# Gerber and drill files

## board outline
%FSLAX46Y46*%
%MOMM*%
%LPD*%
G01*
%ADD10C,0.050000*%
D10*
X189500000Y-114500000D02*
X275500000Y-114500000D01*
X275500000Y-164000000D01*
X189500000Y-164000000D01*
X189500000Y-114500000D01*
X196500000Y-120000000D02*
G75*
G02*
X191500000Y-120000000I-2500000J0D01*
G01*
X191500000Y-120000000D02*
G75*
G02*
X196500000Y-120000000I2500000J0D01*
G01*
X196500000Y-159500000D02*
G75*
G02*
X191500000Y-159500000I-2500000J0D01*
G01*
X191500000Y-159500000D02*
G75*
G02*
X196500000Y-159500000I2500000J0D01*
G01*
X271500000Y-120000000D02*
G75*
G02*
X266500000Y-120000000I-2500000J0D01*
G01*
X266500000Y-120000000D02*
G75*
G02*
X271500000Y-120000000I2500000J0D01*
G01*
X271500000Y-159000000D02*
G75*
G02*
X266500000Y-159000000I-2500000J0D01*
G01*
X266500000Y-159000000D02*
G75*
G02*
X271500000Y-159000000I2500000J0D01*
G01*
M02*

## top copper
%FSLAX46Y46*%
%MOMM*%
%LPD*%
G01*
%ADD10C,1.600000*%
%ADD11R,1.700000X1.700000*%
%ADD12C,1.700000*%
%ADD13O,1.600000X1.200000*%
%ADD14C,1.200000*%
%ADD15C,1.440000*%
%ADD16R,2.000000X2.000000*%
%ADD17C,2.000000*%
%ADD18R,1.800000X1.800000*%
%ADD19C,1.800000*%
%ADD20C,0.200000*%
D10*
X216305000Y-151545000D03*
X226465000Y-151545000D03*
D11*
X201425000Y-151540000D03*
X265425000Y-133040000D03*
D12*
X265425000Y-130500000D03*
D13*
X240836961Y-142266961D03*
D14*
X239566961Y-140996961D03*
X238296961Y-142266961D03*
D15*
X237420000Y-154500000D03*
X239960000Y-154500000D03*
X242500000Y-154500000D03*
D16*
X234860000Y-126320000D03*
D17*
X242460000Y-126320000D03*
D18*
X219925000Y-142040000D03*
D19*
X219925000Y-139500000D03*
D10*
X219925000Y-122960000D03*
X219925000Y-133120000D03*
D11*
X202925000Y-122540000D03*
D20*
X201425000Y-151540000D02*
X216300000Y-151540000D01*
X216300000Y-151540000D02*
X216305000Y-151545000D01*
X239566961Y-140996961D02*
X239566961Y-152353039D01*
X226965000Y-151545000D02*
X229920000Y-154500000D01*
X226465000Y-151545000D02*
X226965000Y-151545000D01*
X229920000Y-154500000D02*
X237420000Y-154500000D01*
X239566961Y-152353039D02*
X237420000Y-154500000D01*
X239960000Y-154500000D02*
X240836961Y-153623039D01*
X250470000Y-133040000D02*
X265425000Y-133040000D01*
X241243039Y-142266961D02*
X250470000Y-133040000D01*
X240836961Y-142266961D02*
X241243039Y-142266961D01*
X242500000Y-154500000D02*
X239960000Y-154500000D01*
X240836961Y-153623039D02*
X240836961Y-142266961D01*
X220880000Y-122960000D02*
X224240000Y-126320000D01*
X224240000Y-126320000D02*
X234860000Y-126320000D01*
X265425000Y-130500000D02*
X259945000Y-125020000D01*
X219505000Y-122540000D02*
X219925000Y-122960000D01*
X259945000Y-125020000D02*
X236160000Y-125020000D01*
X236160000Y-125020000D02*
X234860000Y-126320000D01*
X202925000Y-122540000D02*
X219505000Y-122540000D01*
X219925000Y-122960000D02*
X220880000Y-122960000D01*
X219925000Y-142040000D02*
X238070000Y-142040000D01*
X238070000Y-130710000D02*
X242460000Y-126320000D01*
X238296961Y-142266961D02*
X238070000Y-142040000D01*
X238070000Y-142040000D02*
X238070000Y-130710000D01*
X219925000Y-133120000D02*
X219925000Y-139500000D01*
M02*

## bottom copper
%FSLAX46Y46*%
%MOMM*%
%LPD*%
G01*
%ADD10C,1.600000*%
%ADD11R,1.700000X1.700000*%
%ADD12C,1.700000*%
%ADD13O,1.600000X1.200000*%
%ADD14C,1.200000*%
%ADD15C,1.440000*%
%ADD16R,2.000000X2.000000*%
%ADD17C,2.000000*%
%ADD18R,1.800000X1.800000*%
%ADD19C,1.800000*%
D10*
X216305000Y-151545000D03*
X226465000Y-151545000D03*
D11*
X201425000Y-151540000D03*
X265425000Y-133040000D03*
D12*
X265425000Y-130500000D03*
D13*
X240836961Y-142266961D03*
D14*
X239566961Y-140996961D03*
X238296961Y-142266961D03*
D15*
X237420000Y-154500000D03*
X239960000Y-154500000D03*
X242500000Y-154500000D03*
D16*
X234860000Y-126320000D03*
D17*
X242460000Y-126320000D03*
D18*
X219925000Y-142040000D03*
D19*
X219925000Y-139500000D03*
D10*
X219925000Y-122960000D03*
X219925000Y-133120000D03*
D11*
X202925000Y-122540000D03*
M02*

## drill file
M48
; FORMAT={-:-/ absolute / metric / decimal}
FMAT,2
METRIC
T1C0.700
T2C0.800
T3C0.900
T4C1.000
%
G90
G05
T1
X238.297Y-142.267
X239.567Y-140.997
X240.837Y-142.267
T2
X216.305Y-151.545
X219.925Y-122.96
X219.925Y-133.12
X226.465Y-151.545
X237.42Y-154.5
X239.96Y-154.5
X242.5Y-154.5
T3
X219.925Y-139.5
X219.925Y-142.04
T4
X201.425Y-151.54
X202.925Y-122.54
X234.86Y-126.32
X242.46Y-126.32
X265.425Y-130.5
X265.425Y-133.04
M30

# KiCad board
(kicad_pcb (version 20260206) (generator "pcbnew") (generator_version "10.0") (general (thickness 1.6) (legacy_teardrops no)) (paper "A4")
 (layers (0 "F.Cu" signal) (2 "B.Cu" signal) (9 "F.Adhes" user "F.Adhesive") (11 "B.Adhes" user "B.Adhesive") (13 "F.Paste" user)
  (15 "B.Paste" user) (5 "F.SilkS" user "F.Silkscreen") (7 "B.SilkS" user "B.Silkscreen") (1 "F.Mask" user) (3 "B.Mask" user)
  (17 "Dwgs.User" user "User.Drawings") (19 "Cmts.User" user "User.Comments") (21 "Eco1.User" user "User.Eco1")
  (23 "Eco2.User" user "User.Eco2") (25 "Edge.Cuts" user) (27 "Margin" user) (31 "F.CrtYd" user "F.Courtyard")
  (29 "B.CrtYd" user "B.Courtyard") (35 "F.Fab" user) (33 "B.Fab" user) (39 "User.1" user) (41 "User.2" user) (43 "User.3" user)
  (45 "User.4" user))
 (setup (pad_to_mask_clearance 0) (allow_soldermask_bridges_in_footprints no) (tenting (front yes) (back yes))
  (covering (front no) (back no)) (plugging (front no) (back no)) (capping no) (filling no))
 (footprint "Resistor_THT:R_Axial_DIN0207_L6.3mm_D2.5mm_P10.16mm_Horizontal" (layer "F.Cu") (at 216.305 151.545)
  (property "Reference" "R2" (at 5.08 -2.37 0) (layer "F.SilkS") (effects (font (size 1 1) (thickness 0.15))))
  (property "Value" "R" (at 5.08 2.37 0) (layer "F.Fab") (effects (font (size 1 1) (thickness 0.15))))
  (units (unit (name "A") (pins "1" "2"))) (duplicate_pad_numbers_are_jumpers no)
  (pad "1" thru_hole circle (at 0 0) (size 1.6 1.6) (drill 0.8) (layers "*.Cu" "*.Mask") (remove_unused_layers no) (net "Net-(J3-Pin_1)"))
  (pad "2" thru_hole circle (at 10.16 0) (size 1.6 1.6) (drill 0.8) (layers "*.Cu" "*.Mask") (remove_unused_layers no) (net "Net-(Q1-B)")))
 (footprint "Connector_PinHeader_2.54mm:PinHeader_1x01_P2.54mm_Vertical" (layer "F.Cu") (at 201.425 151.54)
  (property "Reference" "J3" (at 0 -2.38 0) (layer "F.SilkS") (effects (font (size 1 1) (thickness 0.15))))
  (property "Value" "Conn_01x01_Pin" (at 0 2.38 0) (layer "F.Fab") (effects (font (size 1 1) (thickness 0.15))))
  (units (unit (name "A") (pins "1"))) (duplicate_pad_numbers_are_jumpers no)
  (pad "1" thru_hole rect (at 0 0) (size 1.7 1.7) (drill 1) (layers "*.Cu" "*.Mask") (remove_unused_layers no) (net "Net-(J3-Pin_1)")))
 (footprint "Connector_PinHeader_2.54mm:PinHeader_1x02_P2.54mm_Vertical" (layer "F.Cu") (at 265.425 133.04 180)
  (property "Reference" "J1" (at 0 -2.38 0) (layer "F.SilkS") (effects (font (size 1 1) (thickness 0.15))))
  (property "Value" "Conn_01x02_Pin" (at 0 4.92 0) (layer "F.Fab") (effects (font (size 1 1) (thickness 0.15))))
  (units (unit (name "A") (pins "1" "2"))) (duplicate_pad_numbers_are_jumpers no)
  (pad "1" thru_hole rect (at 0 0 180) (size 1.7 1.7) (drill 1) (layers "*.Cu" "*.Mask") (remove_unused_layers no) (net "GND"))
  (pad "2" thru_hole circle (at 0 2.54 180) (size 1.7 1.7) (drill 1) (layers "*.Cu" "*.Mask") (remove_unused_layers no) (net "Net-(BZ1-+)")))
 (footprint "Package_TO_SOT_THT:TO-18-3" (layer "F.Cu") (at 240.836961 142.266961 180)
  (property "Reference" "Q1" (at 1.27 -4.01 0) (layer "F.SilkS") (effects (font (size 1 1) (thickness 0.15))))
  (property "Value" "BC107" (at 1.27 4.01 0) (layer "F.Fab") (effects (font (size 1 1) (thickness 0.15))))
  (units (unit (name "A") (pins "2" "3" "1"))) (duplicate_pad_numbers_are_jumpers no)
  (pad "1" thru_hole oval (at 0 0 180) (size 1.6 1.2) (drill 0.7) (layers "*.Cu" "*.Mask") (remove_unused_layers no) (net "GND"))
  (pad "2" thru_hole circle (at 1.27 1.27 180) (size 1.2 1.2) (drill 0.7) (layers "*.Cu" "*.Mask") (remove_unused_layers no)
   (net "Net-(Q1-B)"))
  (pad "3" thru_hole circle (at 2.54 0 180) (size 1.2 1.2) (drill 0.7) (layers "*.Cu" "*.Mask") (remove_unused_layers no)
   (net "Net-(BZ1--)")))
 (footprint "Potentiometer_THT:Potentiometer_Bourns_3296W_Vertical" (layer "F.Cu") (at 237.42 154.5 180)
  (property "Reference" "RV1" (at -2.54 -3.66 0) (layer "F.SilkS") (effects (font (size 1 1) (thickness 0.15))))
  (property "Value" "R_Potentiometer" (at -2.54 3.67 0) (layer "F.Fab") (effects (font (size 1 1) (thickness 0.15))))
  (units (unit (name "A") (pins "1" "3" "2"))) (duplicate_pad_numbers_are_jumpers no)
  (pad "1" thru_hole circle (at 0 0 180) (size 1.44 1.44) (drill 0.8) (layers "*.Cu" "*.Mask") (remove_unused_layers no) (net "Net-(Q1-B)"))
  (pad "2" thru_hole circle (at -2.54 0 180) (size 1.44 1.44) (drill 0.8) (layers "*.Cu" "*.Mask") (remove_unused_layers no) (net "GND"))
  (pad "3" thru_hole circle (at -5.08 0 180) (size 1.44 1.44) (drill 0.8) (layers "*.Cu" "*.Mask") (remove_unused_layers no) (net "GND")))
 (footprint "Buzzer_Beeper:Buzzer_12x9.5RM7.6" (layer "F.Cu") (at 234.86 126.32)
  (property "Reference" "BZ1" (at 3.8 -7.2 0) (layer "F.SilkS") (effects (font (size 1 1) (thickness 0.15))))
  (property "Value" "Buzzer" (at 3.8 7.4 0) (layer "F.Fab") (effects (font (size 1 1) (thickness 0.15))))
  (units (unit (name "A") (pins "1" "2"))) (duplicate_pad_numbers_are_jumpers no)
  (pad "1" thru_hole rect (at 0 0) (size 2 2) (drill 1) (layers "*.Cu" "*.Mask") (remove_unused_layers no) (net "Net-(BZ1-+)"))
  (pad "2" thru_hole circle (at 7.6 0) (size 2 2) (drill 1) (layers "*.Cu" "*.Mask") (remove_unused_layers no) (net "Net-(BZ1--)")))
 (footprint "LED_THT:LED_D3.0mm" (layer "F.Cu") (at 219.925 142.04 90)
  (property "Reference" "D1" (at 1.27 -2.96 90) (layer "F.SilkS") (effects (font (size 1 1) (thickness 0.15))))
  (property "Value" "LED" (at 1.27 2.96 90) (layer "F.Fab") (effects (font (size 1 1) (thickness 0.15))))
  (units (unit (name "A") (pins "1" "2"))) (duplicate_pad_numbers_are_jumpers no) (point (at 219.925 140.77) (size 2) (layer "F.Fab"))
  (pad "1" thru_hole rect (at 0 0 90) (size 1.8 1.8) (drill 0.9) (layers "*.Cu" "*.Mask") (remove_unused_layers no) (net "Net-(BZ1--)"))
  (pad "2" thru_hole circle (at 2.54 0 90) (size 1.8 1.8) (drill 0.9) (layers "*.Cu" "*.Mask") (remove_unused_layers no) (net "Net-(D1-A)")))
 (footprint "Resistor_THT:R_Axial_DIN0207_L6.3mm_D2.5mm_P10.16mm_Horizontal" (layer "F.Cu") (at 219.925 122.96 -90)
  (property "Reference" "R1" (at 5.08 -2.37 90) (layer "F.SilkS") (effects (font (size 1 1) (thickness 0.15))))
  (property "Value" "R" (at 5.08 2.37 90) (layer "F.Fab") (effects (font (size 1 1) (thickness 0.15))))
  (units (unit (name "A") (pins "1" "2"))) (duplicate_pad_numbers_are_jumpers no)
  (pad "1" thru_hole circle (at 0 0 270) (size 1.6 1.6) (drill 0.8) (layers "*.Cu" "*.Mask") (remove_unused_layers no) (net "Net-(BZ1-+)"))
  (pad "2" thru_hole circle (at 10.16 0 270) (size 1.6 1.6) (drill 0.8) (layers "*.Cu" "*.Mask") (remove_unused_layers no)
   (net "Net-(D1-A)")))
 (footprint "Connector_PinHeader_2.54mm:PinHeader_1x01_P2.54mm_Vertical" (layer "F.Cu") (at 202.925 122.54)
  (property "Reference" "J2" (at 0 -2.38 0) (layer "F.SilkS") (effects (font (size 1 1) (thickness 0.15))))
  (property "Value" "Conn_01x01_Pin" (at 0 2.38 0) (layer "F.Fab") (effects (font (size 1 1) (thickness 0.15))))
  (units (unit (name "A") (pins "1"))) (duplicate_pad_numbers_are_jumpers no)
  (pad "1" thru_hole rect (at 0 0) (size 1.7 1.7) (drill 1) (layers "*.Cu" "*.Mask") (remove_unused_layers no) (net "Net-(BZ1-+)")))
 (gr_rect (start 189.5 114.5) (end 275.5 164) (stroke (width 0.05) (type default)) (fill no) (layer "Edge.Cuts"))
 (gr_circle (center 194 120) (end 196.5 120) (stroke (width 0.05) (type solid)) (fill no) (layer "Edge.Cuts"))
 (gr_circle (center 194 159.5) (end 196.5 159.5) (stroke (width 0.05) (type solid)) (fill no) (layer "Edge.Cuts"))
 (gr_circle (center 269 120) (end 271.5 120) (stroke (width 0.05) (type solid)) (fill no) (layer "Edge.Cuts"))
 (gr_circle (center 269 159) (end 271.5 159) (stroke (width 0.05) (type solid)) (fill no) (layer "Edge.Cuts"))
 (segment (start 201.425 151.54) (end 216.3 151.54) (width 0.2) (layer "F.Cu") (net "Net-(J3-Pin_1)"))
 (segment (start 216.3 151.54) (end 216.305 151.545) (width 0.2) (layer "F.Cu") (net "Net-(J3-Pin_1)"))
 (segment (start 239.566961 140.996961) (end 239.566961 152.353039) (width 0.2) (layer "F.Cu") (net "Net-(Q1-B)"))
 (segment (start 226.965 151.545) (end 229.92 154.5) (width 0.2) (layer "F.Cu") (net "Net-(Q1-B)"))
 (segment (start 226.465 151.545) (end 226.965 151.545) (width 0.2) (layer "F.Cu") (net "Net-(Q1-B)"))
 (segment (start 229.92 154.5) (end 237.42 154.5) (width 0.2) (layer "F.Cu") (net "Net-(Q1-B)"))
 (segment (start 239.566961 152.353039) (end 237.42 154.5) (width 0.2) (layer "F.Cu") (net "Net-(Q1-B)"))
 (segment (start 239.96 154.5) (end 240.836961 153.623039) (width 0.2) (layer "F.Cu") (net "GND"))
 (segment (start 250.47 133.04) (end 265.425 133.04) (width 0.2) (layer "F.Cu") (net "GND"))
 (segment (start 241.243039 142.266961) (end 250.47 133.04) (width 0.2) (layer "F.Cu") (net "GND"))
 (segment (start 240.836961 142.266961) (end 241.243039 142.266961) (width 0.2) (layer "F.Cu") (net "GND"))
 (segment (start 242.5 154.5) (end 239.96 154.5) (width 0.2) (layer "F.Cu") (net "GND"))
 (segment (start 240.836961 153.623039) (end 240.836961 142.266961) (width 0.2) (layer "F.Cu") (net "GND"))
 (segment (start 220.88 122.96) (end 224.24 126.32) (width 0.2) (layer "F.Cu") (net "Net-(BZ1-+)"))
 (segment (start 224.24 126.32) (end 234.86 126.32) (width 0.2) (layer "F.Cu") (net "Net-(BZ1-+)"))
 (segment (start 265.425 130.5) (end 259.945 125.02) (width 0.2) (layer "F.Cu") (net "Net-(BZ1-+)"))
 (segment (start 219.505 122.54) (end 219.925 122.96) (width 0.2) (layer "F.Cu") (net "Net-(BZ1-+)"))
 (segment (start 259.945 125.02) (end 236.16 125.02) (width 0.2) (layer "F.Cu") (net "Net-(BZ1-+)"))
 (segment (start 236.16 125.02) (end 234.86 126.32) (width 0.2) (layer "F.Cu") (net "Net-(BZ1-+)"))
 (segment (start 202.925 122.54) (end 219.505 122.54) (width 0.2) (layer "F.Cu") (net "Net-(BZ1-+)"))
 (segment (start 219.925 122.96) (end 220.88 122.96) (width 0.2) (layer "F.Cu") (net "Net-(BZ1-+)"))
 (segment (start 219.925 142.04) (end 238.07 142.04) (width 0.2) (layer "F.Cu") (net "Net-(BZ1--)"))
 (segment (start 238.07 130.71) (end 242.46 126.32) (width 0.2) (layer "F.Cu") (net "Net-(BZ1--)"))
 (segment (start 238.296961 142.266961) (end 238.07 142.04) (width 0.2) (layer "F.Cu") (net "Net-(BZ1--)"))
 (segment (start 238.07 142.04) (end 238.07 130.71) (width 0.2) (layer "F.Cu") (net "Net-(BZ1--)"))
 (segment (start 219.925 133.12) (end 219.925 139.5) (width 0.2) (layer "F.Cu") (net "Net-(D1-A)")))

